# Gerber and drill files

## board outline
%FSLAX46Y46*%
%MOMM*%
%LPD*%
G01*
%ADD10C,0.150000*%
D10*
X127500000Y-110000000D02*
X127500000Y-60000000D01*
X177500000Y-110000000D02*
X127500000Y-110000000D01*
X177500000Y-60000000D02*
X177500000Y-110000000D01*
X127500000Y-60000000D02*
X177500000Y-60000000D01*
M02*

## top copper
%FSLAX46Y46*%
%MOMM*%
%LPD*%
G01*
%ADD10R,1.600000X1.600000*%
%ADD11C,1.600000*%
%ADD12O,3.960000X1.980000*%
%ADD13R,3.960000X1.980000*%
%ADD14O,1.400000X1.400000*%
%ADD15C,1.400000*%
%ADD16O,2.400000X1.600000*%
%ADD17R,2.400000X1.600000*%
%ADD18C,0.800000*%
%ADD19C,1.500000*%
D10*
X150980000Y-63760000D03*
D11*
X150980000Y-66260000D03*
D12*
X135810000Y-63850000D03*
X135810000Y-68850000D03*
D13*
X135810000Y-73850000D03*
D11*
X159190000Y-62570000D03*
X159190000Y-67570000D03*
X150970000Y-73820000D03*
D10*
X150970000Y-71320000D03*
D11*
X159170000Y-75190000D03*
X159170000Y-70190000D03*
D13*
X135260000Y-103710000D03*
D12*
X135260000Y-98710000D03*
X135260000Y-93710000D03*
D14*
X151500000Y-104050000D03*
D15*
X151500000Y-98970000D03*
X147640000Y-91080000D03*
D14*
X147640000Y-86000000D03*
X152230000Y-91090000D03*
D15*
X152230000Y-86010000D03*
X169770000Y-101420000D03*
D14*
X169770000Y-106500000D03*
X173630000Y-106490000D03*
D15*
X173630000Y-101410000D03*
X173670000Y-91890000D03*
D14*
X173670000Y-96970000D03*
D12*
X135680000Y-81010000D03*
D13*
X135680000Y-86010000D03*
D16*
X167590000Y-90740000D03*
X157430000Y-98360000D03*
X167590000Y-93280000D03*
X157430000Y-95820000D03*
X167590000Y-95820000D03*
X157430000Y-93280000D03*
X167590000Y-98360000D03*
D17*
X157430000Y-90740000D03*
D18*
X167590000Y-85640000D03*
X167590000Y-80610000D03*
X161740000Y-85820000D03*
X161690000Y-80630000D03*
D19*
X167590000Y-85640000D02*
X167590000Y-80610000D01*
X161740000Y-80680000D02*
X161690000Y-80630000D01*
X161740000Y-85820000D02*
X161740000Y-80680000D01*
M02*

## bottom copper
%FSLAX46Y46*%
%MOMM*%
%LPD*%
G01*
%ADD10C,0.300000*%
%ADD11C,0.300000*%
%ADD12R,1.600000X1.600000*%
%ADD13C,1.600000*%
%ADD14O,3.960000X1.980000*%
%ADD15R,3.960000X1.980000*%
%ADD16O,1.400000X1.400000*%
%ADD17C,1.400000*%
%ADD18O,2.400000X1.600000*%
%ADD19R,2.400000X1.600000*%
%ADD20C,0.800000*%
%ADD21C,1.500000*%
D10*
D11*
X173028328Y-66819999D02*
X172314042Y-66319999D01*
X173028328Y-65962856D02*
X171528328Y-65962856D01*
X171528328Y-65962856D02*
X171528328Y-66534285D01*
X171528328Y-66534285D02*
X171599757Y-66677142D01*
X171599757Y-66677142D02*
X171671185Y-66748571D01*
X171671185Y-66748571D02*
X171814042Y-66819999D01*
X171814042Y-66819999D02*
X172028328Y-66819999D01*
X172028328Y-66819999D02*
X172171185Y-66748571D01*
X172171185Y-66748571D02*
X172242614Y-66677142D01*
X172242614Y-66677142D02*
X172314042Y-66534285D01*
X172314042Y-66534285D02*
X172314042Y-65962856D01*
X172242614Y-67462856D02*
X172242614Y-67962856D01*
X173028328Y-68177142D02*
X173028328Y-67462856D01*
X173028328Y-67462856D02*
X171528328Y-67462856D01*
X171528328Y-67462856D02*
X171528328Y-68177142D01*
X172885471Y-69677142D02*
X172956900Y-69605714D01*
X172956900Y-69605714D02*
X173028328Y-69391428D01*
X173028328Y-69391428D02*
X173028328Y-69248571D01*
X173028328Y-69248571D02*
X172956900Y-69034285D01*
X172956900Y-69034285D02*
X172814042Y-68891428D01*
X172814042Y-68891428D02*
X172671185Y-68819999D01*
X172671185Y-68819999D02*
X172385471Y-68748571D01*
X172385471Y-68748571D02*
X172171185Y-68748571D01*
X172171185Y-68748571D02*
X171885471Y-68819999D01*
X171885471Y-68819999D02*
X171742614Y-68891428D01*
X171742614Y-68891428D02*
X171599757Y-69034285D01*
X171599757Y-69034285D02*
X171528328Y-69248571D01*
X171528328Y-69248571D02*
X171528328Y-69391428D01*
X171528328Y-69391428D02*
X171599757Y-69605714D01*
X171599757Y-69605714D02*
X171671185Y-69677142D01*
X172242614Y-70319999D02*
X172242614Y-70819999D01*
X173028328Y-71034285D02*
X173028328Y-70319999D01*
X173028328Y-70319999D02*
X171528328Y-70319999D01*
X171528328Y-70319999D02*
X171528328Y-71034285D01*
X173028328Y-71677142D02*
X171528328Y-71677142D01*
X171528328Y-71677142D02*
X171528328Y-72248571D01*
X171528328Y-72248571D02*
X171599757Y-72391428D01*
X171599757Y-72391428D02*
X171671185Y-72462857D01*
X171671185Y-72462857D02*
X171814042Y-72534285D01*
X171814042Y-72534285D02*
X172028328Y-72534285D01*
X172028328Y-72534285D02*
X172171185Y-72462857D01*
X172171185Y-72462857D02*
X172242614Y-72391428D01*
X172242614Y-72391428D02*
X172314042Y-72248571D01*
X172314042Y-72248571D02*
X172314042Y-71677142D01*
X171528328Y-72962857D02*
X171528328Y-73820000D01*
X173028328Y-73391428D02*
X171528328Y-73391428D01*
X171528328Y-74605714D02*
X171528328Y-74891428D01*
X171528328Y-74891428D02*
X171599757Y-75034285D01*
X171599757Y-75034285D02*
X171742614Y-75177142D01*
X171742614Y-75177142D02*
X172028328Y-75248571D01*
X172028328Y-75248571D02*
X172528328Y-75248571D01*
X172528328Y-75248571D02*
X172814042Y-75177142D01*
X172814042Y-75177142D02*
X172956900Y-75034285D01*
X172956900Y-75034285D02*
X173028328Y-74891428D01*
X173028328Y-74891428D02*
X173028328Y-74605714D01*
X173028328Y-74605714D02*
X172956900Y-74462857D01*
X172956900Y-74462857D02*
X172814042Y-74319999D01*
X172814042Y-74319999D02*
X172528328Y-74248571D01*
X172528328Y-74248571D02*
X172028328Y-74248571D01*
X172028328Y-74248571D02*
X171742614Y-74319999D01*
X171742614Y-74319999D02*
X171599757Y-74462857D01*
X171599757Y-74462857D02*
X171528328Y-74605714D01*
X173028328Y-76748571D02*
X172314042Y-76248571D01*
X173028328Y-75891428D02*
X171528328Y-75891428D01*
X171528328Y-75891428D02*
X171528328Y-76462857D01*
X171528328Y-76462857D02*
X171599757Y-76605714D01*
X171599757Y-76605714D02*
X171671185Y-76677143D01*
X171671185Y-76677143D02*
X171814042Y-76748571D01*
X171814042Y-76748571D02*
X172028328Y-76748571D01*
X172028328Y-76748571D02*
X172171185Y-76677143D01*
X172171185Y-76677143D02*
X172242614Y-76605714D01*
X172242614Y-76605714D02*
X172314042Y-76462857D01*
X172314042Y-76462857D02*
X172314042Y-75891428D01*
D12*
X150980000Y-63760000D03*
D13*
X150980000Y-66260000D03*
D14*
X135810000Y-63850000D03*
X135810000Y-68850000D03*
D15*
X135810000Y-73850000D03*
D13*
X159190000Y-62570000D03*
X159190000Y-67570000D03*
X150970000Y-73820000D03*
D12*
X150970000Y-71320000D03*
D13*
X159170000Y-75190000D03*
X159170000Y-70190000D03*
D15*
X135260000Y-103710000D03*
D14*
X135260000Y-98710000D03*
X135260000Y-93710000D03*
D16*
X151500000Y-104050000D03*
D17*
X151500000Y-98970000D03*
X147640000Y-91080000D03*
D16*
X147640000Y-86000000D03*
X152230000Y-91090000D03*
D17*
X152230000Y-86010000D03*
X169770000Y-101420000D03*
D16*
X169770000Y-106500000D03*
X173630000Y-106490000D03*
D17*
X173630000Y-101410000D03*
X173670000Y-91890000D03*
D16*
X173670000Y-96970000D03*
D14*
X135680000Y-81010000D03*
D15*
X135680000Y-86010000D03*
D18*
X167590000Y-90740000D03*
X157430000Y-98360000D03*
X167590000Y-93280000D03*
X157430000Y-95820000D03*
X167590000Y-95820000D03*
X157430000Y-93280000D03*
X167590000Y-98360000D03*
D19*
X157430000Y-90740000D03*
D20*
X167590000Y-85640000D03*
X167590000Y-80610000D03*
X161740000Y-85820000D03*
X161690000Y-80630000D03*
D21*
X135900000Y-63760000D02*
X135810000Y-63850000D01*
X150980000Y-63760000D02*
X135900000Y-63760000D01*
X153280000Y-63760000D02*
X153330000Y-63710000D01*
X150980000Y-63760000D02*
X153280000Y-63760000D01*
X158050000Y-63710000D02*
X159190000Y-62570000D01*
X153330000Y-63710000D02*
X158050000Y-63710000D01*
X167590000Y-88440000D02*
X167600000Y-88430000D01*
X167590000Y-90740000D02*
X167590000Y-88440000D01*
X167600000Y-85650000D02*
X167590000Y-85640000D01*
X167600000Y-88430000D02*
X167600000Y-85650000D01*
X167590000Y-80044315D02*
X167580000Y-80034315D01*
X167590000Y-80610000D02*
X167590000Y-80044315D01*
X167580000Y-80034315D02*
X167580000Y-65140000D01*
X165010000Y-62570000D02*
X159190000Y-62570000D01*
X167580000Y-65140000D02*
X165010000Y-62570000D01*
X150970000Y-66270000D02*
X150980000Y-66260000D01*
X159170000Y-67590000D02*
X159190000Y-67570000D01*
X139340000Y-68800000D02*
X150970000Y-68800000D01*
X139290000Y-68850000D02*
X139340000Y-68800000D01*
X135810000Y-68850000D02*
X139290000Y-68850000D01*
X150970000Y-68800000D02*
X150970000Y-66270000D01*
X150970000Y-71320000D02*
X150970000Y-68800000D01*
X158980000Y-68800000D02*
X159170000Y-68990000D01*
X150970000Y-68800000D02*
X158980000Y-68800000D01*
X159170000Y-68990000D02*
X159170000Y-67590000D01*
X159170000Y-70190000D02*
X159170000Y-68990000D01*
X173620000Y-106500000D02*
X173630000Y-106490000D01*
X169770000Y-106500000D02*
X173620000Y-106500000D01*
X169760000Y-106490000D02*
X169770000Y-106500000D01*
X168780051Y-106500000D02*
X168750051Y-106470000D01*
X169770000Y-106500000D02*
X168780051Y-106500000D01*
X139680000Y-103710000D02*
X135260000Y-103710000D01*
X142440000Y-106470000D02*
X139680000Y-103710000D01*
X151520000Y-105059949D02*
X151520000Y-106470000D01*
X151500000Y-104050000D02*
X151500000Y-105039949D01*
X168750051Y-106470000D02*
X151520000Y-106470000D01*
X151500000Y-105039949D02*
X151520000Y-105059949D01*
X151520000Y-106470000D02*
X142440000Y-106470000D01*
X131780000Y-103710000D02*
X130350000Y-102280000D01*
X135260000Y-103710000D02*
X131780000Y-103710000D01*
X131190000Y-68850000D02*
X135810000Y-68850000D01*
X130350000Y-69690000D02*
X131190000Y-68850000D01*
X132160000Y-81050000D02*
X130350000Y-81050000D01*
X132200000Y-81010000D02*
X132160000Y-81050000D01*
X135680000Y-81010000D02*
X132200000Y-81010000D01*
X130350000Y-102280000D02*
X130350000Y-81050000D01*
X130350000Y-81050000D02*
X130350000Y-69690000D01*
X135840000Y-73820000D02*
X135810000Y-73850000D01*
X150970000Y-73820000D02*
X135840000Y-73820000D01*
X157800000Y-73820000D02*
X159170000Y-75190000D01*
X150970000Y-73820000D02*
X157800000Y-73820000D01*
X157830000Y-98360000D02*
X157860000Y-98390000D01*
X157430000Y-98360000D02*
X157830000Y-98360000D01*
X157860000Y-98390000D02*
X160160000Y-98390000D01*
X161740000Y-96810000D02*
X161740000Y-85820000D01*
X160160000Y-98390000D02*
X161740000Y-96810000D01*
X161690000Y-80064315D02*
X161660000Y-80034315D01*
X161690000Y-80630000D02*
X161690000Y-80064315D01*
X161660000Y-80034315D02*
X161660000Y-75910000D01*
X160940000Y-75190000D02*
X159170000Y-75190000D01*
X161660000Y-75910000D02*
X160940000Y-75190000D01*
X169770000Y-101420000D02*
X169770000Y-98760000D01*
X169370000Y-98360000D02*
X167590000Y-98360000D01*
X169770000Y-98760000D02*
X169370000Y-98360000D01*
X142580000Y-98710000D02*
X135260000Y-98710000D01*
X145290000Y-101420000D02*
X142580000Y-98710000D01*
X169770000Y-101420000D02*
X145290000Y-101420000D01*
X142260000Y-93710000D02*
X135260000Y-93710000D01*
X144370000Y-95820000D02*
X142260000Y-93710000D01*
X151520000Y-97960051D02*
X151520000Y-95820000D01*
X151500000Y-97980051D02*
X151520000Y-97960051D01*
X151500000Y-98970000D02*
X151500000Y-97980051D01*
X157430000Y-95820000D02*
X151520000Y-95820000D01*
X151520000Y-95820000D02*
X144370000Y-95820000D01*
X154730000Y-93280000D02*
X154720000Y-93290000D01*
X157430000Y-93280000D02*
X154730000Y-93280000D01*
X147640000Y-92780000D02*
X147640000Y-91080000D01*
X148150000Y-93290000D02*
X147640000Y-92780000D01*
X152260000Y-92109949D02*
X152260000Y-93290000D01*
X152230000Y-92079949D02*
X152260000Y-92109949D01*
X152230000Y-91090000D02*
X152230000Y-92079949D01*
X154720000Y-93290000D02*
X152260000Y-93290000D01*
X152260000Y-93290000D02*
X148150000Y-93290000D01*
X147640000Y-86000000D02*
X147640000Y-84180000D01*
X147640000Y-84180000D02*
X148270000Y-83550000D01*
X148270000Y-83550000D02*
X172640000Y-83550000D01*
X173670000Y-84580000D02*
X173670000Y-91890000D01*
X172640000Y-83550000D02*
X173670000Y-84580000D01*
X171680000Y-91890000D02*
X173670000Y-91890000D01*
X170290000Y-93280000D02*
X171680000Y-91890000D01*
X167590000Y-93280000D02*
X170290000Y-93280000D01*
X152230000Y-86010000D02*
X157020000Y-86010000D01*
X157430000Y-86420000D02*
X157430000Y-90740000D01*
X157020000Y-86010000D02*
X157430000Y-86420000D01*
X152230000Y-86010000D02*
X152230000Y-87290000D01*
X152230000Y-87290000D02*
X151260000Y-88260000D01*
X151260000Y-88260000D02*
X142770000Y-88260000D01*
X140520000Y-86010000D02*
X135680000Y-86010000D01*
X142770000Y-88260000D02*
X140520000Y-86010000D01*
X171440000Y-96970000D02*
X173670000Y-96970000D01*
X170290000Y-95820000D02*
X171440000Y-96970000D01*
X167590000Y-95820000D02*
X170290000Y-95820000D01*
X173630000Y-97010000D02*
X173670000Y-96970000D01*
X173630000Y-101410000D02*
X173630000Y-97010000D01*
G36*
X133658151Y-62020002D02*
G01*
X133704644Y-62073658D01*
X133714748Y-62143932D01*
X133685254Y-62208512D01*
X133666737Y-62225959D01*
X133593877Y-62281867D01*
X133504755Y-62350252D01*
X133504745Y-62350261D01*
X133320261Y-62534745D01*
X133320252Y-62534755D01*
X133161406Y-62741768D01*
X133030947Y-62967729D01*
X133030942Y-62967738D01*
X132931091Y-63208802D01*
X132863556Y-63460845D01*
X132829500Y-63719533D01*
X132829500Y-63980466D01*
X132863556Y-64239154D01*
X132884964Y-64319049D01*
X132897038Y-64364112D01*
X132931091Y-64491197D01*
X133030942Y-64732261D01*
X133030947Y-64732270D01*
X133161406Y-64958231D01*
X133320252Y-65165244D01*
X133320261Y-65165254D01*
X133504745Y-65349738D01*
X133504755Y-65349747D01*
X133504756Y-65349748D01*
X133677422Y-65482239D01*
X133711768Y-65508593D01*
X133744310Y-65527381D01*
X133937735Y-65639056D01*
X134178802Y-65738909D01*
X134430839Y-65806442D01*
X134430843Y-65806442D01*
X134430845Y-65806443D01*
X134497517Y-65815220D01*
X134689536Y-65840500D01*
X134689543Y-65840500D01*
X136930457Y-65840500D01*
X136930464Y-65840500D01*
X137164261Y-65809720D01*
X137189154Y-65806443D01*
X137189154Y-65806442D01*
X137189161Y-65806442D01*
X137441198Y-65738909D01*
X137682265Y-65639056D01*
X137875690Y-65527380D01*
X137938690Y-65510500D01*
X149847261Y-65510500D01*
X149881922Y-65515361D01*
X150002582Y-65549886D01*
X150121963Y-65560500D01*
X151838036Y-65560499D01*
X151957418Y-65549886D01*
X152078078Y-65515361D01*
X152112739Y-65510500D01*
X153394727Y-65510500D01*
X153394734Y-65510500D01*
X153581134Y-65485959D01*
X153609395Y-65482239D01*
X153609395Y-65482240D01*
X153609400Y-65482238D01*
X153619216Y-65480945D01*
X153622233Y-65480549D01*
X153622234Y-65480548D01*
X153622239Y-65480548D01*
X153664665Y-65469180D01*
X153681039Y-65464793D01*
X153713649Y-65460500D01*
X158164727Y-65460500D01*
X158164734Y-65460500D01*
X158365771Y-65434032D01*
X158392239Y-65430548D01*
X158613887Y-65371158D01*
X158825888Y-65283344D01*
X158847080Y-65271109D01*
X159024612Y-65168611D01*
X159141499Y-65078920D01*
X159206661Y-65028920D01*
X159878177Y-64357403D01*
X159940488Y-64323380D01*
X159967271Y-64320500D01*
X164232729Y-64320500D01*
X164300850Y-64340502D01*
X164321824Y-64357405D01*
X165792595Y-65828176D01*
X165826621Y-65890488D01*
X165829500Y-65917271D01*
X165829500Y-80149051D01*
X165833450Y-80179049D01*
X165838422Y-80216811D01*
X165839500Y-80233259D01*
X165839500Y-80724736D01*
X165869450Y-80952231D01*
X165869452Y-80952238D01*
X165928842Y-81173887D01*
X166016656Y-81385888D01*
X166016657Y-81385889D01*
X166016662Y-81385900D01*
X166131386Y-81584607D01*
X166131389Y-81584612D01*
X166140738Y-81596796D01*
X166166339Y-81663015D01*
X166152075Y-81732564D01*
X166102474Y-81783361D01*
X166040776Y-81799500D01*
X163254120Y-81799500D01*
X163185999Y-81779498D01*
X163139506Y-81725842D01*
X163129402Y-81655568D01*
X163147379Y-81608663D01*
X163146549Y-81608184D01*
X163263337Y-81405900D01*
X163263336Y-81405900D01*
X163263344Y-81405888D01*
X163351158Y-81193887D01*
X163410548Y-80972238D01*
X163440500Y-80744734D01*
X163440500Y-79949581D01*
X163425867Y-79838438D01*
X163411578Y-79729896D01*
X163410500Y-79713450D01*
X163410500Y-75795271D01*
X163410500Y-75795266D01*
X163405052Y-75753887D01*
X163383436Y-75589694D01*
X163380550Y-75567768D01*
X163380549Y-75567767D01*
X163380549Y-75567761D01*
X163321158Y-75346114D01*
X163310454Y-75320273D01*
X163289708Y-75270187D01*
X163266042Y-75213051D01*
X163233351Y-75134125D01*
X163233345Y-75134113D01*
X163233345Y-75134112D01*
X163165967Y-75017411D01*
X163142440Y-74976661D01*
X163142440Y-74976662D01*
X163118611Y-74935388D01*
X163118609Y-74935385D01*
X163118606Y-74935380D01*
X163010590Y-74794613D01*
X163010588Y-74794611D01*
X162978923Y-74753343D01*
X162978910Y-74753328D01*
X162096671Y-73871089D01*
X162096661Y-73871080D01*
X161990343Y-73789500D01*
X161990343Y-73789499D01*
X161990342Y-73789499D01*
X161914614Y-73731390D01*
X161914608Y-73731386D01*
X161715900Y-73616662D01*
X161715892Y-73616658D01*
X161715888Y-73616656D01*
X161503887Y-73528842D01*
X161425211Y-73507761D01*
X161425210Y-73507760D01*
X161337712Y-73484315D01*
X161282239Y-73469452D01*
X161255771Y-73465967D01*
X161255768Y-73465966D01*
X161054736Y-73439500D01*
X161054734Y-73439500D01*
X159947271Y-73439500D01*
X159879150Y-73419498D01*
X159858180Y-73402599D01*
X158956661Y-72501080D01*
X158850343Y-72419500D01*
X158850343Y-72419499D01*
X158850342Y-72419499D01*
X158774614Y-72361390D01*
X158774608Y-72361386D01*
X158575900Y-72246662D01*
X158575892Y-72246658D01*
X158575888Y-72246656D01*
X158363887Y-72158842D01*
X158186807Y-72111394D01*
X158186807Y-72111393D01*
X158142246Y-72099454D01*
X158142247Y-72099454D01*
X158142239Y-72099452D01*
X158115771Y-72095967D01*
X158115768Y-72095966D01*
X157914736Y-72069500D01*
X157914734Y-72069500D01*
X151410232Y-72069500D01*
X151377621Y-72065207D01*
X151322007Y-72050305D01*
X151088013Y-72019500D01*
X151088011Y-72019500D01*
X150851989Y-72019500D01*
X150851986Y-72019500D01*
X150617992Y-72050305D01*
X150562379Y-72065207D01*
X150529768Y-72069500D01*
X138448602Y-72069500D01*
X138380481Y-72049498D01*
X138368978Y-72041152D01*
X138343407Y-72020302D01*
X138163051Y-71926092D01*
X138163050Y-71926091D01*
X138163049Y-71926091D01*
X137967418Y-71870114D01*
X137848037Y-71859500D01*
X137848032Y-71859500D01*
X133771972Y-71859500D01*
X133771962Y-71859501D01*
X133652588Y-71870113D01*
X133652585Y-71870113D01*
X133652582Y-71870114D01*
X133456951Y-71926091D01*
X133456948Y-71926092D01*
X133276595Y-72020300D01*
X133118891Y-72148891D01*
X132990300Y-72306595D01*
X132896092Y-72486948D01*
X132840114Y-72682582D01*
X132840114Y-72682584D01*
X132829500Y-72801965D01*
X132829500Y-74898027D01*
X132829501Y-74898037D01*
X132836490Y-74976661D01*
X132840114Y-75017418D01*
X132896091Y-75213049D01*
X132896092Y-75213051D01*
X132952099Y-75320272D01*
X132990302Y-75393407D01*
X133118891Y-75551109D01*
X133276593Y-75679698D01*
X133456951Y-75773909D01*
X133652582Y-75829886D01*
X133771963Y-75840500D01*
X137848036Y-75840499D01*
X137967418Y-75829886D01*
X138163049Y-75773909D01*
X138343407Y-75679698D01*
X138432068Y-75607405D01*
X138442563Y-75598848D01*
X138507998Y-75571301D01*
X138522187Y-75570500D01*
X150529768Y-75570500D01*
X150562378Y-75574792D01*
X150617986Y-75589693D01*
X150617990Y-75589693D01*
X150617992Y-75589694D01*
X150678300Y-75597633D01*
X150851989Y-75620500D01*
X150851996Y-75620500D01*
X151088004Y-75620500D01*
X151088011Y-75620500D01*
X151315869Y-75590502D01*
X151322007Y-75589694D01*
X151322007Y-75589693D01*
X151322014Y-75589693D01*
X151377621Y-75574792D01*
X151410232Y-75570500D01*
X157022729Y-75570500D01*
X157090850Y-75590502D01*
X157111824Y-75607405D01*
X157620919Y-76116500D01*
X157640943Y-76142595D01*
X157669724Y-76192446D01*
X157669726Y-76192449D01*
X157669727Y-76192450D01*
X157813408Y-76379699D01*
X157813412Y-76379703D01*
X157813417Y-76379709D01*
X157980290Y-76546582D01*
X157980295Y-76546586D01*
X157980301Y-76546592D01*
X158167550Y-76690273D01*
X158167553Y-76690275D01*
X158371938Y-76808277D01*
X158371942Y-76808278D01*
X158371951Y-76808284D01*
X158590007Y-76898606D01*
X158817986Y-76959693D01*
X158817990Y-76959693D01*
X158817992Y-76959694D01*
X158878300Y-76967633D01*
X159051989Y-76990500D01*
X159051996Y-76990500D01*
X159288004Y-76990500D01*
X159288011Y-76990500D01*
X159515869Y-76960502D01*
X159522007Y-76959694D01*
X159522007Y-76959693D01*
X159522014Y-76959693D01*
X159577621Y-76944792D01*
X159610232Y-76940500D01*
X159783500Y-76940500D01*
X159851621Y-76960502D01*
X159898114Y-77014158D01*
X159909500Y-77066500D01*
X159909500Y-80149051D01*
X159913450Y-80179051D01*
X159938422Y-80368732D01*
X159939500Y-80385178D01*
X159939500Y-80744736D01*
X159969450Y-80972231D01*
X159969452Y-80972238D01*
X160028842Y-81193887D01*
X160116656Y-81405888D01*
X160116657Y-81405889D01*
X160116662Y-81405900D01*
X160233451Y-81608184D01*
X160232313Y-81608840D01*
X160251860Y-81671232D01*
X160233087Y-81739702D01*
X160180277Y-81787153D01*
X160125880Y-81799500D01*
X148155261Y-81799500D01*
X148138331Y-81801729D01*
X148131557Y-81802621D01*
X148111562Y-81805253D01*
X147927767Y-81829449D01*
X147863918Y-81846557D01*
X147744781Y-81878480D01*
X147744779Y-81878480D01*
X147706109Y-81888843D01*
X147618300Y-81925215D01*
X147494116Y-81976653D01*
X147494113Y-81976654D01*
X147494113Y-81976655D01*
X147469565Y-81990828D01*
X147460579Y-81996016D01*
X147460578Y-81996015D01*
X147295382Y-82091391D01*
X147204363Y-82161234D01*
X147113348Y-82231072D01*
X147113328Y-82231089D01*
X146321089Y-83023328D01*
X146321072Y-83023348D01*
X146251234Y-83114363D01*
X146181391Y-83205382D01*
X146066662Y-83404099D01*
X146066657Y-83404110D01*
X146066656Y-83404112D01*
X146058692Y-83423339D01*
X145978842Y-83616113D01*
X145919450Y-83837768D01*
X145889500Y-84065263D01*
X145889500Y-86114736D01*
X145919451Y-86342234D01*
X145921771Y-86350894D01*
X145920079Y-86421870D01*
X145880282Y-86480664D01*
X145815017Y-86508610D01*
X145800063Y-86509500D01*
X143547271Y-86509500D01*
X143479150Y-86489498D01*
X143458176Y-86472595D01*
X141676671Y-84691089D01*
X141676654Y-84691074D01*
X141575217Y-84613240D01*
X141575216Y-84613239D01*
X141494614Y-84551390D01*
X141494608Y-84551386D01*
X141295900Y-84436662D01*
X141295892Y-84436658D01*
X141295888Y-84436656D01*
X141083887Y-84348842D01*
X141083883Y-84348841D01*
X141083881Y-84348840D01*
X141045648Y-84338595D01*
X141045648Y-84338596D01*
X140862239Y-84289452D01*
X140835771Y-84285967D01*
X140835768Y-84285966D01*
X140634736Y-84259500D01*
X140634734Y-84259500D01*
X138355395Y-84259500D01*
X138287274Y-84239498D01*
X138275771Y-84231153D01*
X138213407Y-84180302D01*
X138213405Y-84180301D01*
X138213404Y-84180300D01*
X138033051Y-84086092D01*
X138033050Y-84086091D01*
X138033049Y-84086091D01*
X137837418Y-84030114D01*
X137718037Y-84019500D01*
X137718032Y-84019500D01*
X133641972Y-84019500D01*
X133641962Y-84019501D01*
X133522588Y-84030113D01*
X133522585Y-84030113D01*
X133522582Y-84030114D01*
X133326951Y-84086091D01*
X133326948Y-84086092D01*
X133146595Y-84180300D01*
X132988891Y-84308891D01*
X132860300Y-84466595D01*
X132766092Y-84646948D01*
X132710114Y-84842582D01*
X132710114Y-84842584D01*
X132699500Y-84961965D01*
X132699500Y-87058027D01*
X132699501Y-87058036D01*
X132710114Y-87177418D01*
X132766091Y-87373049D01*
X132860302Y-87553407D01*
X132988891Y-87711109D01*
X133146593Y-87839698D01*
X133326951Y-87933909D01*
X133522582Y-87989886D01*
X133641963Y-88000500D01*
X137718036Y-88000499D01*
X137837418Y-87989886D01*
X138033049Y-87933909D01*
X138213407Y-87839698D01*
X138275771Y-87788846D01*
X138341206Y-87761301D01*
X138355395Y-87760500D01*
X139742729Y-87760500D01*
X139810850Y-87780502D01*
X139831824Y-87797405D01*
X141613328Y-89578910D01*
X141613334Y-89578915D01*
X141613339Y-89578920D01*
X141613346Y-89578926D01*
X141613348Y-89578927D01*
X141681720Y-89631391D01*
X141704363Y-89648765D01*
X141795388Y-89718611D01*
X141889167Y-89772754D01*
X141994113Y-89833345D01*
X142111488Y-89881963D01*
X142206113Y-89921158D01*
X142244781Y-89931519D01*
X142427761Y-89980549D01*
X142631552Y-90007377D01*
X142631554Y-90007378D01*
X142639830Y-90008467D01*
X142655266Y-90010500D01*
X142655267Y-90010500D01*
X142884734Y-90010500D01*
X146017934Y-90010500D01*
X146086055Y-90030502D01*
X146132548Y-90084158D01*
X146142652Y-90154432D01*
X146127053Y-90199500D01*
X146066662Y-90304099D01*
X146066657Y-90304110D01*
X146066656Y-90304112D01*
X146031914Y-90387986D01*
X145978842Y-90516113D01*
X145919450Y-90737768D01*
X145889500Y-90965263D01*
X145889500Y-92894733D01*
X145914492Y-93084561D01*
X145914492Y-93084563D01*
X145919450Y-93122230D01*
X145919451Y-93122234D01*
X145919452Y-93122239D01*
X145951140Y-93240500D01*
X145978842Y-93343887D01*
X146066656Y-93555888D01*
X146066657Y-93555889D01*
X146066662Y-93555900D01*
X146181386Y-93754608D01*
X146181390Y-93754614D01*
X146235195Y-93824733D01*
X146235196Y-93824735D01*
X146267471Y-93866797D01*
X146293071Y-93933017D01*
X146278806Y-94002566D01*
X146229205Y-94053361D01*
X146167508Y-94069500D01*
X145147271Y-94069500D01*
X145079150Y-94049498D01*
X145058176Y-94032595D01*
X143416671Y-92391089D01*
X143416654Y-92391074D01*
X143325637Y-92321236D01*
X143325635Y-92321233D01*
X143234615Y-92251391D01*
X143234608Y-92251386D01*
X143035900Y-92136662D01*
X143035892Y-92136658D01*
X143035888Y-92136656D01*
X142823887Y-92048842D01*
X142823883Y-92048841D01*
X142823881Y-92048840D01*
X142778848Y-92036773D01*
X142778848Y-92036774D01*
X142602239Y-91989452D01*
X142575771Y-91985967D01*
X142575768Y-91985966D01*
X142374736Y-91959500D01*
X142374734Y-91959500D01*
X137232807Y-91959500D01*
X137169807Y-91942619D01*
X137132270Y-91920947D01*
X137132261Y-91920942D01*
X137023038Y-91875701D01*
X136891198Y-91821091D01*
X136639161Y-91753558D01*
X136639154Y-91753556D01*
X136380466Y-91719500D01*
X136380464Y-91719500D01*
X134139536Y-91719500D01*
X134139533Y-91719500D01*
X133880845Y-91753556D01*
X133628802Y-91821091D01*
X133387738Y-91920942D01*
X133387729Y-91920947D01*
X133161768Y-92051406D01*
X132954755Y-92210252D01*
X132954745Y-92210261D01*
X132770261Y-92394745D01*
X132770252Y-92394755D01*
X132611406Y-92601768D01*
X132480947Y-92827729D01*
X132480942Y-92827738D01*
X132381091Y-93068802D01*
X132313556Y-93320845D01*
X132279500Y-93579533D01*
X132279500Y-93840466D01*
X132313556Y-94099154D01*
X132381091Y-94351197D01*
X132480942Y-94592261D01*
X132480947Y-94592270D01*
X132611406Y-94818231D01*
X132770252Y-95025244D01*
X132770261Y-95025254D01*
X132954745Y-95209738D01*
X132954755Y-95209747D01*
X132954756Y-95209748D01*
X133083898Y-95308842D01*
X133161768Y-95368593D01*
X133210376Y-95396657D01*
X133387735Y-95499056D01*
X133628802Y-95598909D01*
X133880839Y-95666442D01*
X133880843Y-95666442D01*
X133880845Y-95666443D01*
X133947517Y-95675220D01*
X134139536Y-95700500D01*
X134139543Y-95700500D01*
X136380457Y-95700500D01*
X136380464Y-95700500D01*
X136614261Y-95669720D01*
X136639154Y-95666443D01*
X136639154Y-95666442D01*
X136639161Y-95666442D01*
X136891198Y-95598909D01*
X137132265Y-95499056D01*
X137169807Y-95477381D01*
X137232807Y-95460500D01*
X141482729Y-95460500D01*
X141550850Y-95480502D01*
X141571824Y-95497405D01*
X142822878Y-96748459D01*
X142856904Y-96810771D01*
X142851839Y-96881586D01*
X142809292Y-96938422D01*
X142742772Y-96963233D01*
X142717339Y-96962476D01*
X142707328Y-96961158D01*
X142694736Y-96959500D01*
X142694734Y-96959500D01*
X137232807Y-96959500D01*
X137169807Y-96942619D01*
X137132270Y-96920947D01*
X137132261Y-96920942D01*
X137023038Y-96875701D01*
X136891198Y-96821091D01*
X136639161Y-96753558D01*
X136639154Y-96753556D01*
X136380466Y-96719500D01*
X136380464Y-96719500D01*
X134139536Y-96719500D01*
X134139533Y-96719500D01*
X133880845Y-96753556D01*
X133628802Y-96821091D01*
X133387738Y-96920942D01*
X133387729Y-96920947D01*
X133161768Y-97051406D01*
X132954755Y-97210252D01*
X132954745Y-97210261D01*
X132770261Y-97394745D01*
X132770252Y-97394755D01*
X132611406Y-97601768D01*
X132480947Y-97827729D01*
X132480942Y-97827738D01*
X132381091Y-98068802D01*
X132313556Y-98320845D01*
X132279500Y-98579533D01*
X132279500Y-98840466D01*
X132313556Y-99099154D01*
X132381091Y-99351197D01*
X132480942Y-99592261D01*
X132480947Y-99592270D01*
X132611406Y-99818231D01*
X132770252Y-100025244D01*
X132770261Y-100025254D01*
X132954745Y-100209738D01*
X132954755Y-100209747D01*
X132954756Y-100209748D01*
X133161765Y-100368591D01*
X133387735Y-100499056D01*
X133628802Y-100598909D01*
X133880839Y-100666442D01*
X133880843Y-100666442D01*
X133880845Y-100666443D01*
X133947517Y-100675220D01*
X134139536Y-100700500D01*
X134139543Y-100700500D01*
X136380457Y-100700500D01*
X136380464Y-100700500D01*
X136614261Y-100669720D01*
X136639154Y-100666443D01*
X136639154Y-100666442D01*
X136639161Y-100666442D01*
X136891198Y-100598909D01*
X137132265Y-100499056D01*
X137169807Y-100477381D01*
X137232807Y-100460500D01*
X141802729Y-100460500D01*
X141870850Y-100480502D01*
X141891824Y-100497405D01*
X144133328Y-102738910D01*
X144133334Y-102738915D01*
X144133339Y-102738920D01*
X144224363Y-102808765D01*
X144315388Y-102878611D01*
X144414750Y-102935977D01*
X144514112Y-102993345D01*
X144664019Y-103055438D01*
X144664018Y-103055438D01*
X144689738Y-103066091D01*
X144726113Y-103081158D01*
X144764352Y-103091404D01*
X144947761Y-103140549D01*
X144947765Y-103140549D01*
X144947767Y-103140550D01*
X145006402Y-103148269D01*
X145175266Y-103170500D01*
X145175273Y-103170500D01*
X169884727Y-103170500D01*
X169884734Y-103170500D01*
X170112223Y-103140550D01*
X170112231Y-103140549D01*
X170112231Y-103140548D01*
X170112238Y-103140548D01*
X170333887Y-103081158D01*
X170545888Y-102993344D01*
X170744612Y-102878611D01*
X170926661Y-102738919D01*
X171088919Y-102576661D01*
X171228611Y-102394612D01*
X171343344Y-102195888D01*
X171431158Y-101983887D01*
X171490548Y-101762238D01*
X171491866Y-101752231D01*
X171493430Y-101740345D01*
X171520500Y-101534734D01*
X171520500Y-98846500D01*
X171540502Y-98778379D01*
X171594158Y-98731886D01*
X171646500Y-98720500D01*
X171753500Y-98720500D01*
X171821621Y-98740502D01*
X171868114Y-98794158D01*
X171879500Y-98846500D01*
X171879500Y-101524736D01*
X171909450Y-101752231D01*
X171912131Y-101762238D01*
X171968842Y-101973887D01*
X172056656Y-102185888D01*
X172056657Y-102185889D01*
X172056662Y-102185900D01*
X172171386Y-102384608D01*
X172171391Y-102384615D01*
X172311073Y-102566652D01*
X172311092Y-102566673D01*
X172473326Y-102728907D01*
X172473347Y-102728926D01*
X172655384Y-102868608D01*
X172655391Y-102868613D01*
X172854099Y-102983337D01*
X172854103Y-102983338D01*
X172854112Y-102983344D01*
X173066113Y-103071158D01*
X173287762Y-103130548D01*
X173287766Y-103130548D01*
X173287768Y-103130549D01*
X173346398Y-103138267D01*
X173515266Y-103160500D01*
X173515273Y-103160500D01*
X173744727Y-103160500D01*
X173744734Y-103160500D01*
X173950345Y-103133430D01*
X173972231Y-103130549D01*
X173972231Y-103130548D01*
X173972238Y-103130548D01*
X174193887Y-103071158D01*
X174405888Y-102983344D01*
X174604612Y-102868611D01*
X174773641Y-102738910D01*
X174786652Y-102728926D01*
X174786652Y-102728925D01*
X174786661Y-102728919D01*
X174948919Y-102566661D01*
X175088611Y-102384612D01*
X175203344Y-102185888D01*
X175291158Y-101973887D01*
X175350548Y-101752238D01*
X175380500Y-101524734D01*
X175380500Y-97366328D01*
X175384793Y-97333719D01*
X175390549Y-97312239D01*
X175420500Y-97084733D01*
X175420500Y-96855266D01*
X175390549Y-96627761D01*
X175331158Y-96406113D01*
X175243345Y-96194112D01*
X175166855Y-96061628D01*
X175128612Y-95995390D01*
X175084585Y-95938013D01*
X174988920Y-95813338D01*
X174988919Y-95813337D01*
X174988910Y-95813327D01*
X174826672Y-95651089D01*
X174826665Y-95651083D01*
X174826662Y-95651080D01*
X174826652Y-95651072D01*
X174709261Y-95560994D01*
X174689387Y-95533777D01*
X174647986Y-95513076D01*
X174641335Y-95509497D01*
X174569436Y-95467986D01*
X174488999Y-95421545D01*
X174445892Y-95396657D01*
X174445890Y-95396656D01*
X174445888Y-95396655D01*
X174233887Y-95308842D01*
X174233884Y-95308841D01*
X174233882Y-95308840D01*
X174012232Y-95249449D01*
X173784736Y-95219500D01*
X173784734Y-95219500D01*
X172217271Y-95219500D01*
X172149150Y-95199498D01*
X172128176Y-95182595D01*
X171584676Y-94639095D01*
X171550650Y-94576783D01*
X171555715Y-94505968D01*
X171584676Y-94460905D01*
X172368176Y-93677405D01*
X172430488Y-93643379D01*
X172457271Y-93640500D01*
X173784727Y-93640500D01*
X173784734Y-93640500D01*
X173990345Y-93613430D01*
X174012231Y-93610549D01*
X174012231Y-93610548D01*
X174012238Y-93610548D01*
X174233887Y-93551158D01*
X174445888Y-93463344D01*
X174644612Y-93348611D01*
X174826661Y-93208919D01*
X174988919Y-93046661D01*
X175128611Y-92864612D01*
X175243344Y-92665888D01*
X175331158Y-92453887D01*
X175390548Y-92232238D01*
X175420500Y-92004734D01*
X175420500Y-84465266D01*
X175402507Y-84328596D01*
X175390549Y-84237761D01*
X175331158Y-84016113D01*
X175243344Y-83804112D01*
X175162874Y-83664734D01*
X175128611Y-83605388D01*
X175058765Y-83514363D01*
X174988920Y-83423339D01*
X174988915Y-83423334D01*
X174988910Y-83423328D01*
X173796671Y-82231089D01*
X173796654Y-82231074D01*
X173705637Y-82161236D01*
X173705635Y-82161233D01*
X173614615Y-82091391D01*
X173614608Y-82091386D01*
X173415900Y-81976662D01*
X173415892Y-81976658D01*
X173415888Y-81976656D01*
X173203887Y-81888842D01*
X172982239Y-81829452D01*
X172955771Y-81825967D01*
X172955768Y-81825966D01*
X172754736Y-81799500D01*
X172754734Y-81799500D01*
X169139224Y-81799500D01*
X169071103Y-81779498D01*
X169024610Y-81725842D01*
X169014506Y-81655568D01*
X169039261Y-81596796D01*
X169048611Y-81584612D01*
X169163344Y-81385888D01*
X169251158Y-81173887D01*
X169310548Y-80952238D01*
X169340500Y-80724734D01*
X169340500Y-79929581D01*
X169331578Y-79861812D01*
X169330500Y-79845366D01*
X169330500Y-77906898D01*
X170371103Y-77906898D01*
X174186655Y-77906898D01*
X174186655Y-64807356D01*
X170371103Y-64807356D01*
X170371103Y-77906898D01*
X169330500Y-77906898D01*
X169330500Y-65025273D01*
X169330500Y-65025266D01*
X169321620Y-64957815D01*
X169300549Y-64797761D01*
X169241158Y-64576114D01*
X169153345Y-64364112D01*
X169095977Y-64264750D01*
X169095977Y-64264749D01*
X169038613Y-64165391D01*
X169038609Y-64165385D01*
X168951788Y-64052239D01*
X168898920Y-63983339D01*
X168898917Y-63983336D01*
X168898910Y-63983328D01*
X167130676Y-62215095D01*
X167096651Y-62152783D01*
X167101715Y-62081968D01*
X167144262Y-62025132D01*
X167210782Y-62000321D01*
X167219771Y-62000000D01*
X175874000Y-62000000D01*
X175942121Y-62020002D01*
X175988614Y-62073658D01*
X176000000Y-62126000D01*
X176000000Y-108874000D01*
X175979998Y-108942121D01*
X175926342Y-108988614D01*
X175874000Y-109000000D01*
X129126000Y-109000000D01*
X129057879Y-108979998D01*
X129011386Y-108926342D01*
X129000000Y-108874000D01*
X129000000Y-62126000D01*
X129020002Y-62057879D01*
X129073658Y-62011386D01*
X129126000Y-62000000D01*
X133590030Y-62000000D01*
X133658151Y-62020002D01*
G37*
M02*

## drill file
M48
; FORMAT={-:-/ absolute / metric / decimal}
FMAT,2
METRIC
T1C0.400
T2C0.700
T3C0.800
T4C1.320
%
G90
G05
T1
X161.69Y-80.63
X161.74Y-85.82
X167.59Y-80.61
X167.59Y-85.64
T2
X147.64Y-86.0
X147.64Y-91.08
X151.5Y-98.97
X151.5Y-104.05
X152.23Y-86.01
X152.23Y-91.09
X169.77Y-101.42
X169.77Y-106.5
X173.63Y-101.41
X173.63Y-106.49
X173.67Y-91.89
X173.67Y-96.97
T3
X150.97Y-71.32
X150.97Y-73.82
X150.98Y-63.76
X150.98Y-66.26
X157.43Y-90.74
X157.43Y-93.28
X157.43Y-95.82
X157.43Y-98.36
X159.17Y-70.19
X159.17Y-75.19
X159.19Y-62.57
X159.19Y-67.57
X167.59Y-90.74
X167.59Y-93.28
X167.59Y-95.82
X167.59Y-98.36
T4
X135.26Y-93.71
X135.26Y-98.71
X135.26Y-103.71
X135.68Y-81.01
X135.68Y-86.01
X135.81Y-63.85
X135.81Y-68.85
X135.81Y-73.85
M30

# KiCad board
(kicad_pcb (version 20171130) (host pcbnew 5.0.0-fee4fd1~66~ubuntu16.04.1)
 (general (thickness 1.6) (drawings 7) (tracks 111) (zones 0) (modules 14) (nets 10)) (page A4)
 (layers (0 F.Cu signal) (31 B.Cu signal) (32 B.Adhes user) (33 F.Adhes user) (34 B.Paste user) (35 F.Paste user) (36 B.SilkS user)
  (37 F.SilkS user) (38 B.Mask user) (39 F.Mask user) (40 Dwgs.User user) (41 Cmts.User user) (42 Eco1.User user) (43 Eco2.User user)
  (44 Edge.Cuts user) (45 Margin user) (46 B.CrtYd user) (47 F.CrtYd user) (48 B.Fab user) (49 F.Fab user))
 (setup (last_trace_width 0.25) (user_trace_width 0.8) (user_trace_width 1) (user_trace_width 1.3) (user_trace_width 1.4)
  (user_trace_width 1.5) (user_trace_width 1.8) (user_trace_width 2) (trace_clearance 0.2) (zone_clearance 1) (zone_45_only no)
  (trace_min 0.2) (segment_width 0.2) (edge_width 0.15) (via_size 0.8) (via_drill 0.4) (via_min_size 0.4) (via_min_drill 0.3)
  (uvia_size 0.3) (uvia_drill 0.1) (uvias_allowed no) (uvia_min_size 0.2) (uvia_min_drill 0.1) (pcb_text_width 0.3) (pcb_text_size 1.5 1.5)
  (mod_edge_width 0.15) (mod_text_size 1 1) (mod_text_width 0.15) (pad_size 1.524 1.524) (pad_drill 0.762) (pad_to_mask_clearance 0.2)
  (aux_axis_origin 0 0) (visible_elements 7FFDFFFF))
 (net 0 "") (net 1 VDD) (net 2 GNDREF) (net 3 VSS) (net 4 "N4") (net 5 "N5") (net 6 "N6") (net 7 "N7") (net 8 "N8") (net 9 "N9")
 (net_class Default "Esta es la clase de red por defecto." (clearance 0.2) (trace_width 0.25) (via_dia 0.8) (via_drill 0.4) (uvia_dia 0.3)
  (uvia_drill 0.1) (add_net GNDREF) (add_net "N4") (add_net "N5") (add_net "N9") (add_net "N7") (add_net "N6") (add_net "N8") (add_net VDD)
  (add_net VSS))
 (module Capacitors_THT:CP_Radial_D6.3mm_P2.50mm (layer F.Cu) (at 150.98 63.76 270)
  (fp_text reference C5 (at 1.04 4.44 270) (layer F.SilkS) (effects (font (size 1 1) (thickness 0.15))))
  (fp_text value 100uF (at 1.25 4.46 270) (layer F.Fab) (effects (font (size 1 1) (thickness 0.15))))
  (pad 1 thru_hole rect (at 0 0 270) (size 1.6 1.6) (drill 0.8) (layers *.Cu *.Mask) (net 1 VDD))
  (pad 2 thru_hole circle (at 2.5 0 270) (size 1.6 1.6) (drill 0.8) (layers *.Cu *.Mask) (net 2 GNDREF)))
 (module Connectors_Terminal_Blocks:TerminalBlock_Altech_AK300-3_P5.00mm (layer F.Cu) (at 135.81 73.85 90)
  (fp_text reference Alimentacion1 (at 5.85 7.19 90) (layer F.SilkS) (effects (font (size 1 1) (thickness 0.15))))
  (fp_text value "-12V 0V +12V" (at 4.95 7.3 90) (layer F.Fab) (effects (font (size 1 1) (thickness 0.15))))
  (pad 3 thru_hole oval (at 10 0 90) (size 1.98 3.96) (drill 1.32) (layers *.Cu *.Mask) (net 1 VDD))
  (pad 2 thru_hole oval (at 5 0 90) (size 1.98 3.96) (drill 1.32) (layers *.Cu *.Mask) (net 2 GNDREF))
  (pad 1 thru_hole rect (at 0 0 90) (size 1.98 3.96) (drill 1.32) (layers *.Cu *.Mask) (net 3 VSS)))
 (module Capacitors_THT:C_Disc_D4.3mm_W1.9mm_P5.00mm (layer F.Cu) (at 159.19 67.57 90)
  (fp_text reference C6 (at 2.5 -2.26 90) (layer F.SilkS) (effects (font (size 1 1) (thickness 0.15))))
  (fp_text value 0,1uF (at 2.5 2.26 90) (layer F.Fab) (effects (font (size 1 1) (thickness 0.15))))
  (pad 2 thru_hole circle (at 5 0 90) (size 1.6 1.6) (drill 0.8) (layers *.Cu *.Mask) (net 1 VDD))
  (pad 1 thru_hole circle (at 0 0 90) (size 1.6 1.6) (drill 0.8) (layers *.Cu *.Mask) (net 2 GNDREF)))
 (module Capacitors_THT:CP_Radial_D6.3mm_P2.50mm (layer F.Cu) (at 150.97 71.32 270)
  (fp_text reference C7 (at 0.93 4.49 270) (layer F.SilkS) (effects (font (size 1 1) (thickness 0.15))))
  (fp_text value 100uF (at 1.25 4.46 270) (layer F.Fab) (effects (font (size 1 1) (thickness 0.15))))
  (pad 2 thru_hole circle (at 2.5 0 270) (size 1.6 1.6) (drill 0.8) (layers *.Cu *.Mask) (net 3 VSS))
  (pad 1 thru_hole rect (at 0 0 270) (size 1.6 1.6) (drill 0.8) (layers *.Cu *.Mask) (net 2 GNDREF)))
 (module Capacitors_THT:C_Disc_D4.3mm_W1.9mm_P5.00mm (layer F.Cu) (at 159.17 75.19 90)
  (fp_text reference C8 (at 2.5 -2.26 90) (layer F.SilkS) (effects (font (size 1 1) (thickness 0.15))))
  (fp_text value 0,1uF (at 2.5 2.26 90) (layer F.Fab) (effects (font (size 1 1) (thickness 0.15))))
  (pad 1 thru_hole circle (at 0 0 90) (size 1.6 1.6) (drill 0.8) (layers *.Cu *.Mask) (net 3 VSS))
  (pad 2 thru_hole circle (at 5 0 90) (size 1.6 1.6) (drill 0.8) (layers *.Cu *.Mask) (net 2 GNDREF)))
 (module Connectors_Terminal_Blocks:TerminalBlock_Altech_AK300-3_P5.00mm (layer F.Cu) (at 135.26 103.71 90)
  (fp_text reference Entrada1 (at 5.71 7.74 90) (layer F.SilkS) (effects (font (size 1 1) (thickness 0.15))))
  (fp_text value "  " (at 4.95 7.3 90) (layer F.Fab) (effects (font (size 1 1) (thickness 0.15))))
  (pad 1 thru_hole rect (at 0 0 90) (size 1.98 3.96) (drill 1.32) (layers *.Cu *.Mask) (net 2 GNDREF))
  (pad 2 thru_hole oval (at 5 0 90) (size 1.98 3.96) (drill 1.32) (layers *.Cu *.Mask) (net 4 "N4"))
  (pad 3 thru_hole oval (at 10 0 90) (size 1.98 3.96) (drill 1.32) (layers *.Cu *.Mask) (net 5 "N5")))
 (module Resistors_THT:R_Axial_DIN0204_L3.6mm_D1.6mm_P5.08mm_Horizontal (layer F.Cu) (at 151.5 98.97 270)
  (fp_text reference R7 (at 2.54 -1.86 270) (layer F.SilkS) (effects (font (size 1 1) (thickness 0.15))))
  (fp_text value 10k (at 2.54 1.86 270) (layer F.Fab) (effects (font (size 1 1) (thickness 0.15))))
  (pad 2 thru_hole oval (at 5.08 0 270) (size 1.4 1.4) (drill 0.7) (layers *.Cu *.Mask) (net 2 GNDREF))
  (pad 1 thru_hole circle (at 0 0 270) (size 1.4 1.4) (drill 0.7) (layers *.Cu *.Mask) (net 5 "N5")))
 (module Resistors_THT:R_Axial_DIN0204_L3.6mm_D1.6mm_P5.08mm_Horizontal (layer F.Cu) (at 147.64 91.08 90)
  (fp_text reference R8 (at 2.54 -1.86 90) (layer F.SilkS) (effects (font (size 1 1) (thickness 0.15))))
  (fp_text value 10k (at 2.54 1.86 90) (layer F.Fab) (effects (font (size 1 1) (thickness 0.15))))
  (pad 1 thru_hole circle (at 0 0 90) (size 1.4 1.4) (drill 0.7) (layers *.Cu *.Mask) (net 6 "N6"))
  (pad 2 thru_hole oval (at 5.08 0 90) (size 1.4 1.4) (drill 0.7) (layers *.Cu *.Mask) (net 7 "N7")))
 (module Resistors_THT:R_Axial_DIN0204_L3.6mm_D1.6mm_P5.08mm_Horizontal (layer F.Cu) (at 152.23 86.01 270)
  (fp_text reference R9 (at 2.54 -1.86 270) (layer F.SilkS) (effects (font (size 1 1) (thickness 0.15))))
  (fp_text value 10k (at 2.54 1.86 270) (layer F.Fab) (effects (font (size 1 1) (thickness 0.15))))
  (pad 2 thru_hole oval (at 5.08 0 270) (size 1.4 1.4) (drill 0.7) (layers *.Cu *.Mask) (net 6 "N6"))
  (pad 1 thru_hole circle (at 0 0 270) (size 1.4 1.4) (drill 0.7) (layers *.Cu *.Mask) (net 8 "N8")))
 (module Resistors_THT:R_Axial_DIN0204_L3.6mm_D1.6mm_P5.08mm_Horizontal (layer F.Cu) (at 169.77 101.42 270)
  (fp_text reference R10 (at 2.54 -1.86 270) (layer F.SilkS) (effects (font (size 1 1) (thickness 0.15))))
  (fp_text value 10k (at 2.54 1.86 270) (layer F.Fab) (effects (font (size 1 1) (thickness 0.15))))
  (pad 1 thru_hole circle (at 0 0 270) (size 1.4 1.4) (drill 0.7) (layers *.Cu *.Mask) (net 4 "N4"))
  (pad 2 thru_hole oval (at 5.08 0 270) (size 1.4 1.4) (drill 0.7) (layers *.Cu *.Mask) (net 2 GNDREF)))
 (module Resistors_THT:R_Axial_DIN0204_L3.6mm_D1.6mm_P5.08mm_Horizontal (layer F.Cu) (at 173.63 101.41 270)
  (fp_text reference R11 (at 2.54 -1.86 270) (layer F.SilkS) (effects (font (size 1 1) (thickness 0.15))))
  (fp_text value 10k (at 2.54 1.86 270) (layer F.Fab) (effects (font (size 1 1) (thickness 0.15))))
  (pad 2 thru_hole oval (at 5.08 0 270) (size 1.4 1.4) (drill 0.7) (layers *.Cu *.Mask) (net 2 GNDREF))
  (pad 1 thru_hole circle (at 0 0 270) (size 1.4 1.4) (drill 0.7) (layers *.Cu *.Mask) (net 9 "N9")))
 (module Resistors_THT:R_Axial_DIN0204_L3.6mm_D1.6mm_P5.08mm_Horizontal (layer F.Cu) (at 173.67 91.89 270)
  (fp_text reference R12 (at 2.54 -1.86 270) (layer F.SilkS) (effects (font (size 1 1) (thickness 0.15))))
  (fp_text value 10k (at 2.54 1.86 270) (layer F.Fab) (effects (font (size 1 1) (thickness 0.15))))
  (pad 1 thru_hole circle (at 0 0 270) (size 1.4 1.4) (drill 0.7) (layers *.Cu *.Mask) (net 7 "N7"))
  (pad 2 thru_hole oval (at 5.08 0 270) (size 1.4 1.4) (drill 0.7) (layers *.Cu *.Mask) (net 9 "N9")))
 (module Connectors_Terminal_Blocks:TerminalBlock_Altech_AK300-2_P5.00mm (layer F.Cu) (at 135.68 86.01 90)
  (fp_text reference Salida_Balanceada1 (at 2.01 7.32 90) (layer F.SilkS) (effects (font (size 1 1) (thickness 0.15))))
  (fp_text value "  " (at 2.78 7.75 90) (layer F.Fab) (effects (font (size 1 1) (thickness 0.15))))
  (pad 2 thru_hole oval (at 5 0 90) (size 1.98 3.96) (drill 1.32) (layers *.Cu *.Mask) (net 2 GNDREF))
  (pad 1 thru_hole rect (at 0 0 90) (size 1.98 3.96) (drill 1.32) (layers *.Cu *.Mask) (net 8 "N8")))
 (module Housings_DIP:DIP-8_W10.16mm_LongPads (layer F.Cu) (at 157.43 90.74)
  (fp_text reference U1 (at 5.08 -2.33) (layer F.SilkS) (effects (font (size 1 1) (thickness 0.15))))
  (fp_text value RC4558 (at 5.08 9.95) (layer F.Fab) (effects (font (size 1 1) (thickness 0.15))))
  (pad 8 thru_hole oval (at 10.16 0) (size 2.4 1.6) (drill 0.8) (layers *.Cu *.Mask) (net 1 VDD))
  (pad 4 thru_hole oval (at 0 7.62) (size 2.4 1.6) (drill 0.8) (layers *.Cu *.Mask) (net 3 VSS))
  (pad 7 thru_hole oval (at 10.16 2.54) (size 2.4 1.6) (drill 0.8) (layers *.Cu *.Mask) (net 7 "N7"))
  (pad 3 thru_hole oval (at 0 5.08) (size 2.4 1.6) (drill 0.8) (layers *.Cu *.Mask) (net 5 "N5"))
  (pad 6 thru_hole oval (at 10.16 5.08) (size 2.4 1.6) (drill 0.8) (layers *.Cu *.Mask) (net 9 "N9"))
  (pad 2 thru_hole oval (at 0 2.54) (size 2.4 1.6) (drill 0.8) (layers *.Cu *.Mask) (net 6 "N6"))
  (pad 5 thru_hole oval (at 10.16 7.62) (size 2.4 1.6) (drill 0.8) (layers *.Cu *.Mask) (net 4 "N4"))
  (pad 1 thru_hole rect (at 0 0) (size 2.4 1.6) (drill 0.8) (layers *.Cu *.Mask) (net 8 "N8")))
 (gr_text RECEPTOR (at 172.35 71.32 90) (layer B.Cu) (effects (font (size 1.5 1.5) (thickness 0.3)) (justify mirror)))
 (gr_line (start 127.5 110) (end 127.5 60) (layer Edge.Cuts) (width 0.15))
 (gr_line (start 177.5 110) (end 127.5 110) (layer Edge.Cuts) (width 0.15))
 (gr_line (start 177.5 60) (end 177.5 110) (layer Edge.Cuts) (width 0.15))
 (gr_line (start 127.5 60) (end 177.5 60) (layer Edge.Cuts) (width 0.15))
 (segment (start 135.9 63.76) (end 135.81 63.85) (width 1.5) (layer B.Cu) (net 1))
 (segment (start 150.98 63.76) (end 135.9 63.76) (width 1.5) (layer B.Cu) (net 1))
 (segment (start 153.28 63.76) (end 153.33 63.71) (width 1.5) (layer B.Cu) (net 1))
 (segment (start 150.98 63.76) (end 153.28 63.76) (width 1.5) (layer B.Cu) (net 1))
 (segment (start 158.05 63.71) (end 159.19 62.57) (width 1.5) (layer B.Cu) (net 1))
 (segment (start 153.33 63.71) (end 158.05 63.71) (width 1.5) (layer B.Cu) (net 1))
 (segment (start 167.59 88.44) (end 167.6 88.43) (width 1.5) (layer B.Cu) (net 1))
 (segment (start 167.59 90.74) (end 167.59 88.44) (width 1.5) (layer B.Cu) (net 1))
 (via (at 167.59 85.64) (size 0.8) (drill 0.4) (layers F.Cu B.Cu) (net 1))
 (segment (start 167.6 85.65) (end 167.59 85.64) (width 1.5) (layer B.Cu) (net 1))
 (segment (start 167.6 88.43) (end 167.6 85.65) (width 1.5) (layer B.Cu) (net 1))
 (segment (start 167.59 85.64) (end 167.59 80.61) (width 1.5) (layer F.Cu) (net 1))
 (via (at 167.59 80.61) (size 0.8) (drill 0.4) (layers F.Cu B.Cu) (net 1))
 (segment (start 167.59 80.044315) (end 167.58 80.034315) (width 1.5) (layer B.Cu) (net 1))
 (segment (start 167.59 80.61) (end 167.59 80.044315) (width 1.5) (layer B.Cu) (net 1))
 (segment (start 167.58 80.034315) (end 167.58 65.14) (width 1.5) (layer B.Cu) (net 1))
 (segment (start 165.01 62.57) (end 159.19 62.57) (width 1.5) (layer B.Cu) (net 1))
 (segment (start 167.58 65.14) (end 165.01 62.57) (width 1.5) (layer B.Cu) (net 1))
 (segment (start 150.97 66.27) (end 150.98 66.26) (width 1.5) (layer B.Cu) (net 2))
 (segment (start 159.17 67.59) (end 159.19 67.57) (width 1.5) (layer B.Cu) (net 2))
 (segment (start 139.34 68.8) (end 150.97 68.8) (width 1.5) (layer B.Cu) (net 2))
 (segment (start 139.29 68.85) (end 139.34 68.8) (width 1.5) (layer B.Cu) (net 2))
 (segment (start 135.81 68.85) (end 139.29 68.85) (width 1.5) (layer B.Cu) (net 2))
 (segment (start 150.97 68.8) (end 150.97 66.27) (width 1.5) (layer B.Cu) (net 2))
 (segment (start 150.97 71.32) (end 150.97 68.8) (width 1.5) (layer B.Cu) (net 2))
 (segment (start 158.98 68.8) (end 159.17 68.99) (width 1.5) (layer B.Cu) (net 2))
 (segment (start 150.97 68.8) (end 158.98 68.8) (width 1.5) (layer B.Cu) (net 2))
 (segment (start 159.17 68.99) (end 159.17 67.59) (width 1.5) (layer B.Cu) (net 2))
 (segment (start 159.17 70.19) (end 159.17 68.99) (width 1.5) (layer B.Cu) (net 2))
 (segment (start 173.62 106.5) (end 173.63 106.49) (width 1.5) (layer B.Cu) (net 2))
 (segment (start 169.77 106.5) (end 173.62 106.5) (width 1.5) (layer B.Cu) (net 2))
 (segment (start 169.76 106.49) (end 169.77 106.5) (width 1.5) (layer B.Cu) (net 2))
 (segment (start 168.780051 106.5) (end 168.750051 106.47) (width 1.5) (layer B.Cu) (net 2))
 (segment (start 169.77 106.5) (end 168.780051 106.5) (width 1.5) (layer B.Cu) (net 2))
 (segment (start 139.68 103.71) (end 135.26 103.71) (width 1.5) (layer B.Cu) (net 2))
 (segment (start 142.44 106.47) (end 139.68 103.71) (width 1.5) (layer B.Cu) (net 2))
 (segment (start 151.52 105.059949) (end 151.52 106.47) (width 1.5) (layer B.Cu) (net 2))
 (segment (start 151.5 104.05) (end 151.5 105.039949) (width 1.5) (layer B.Cu) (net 2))
 (segment (start 168.750051 106.47) (end 151.52 106.47) (width 1.5) (layer B.Cu) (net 2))
 (segment (start 151.5 105.039949) (end 151.52 105.059949) (width 1.5) (layer B.Cu) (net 2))
 (segment (start 151.52 106.47) (end 142.44 106.47) (width 1.5) (layer B.Cu) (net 2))
 (segment (start 131.78 103.71) (end 130.35 102.28) (width 1.5) (layer B.Cu) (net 2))
 (segment (start 135.26 103.71) (end 131.78 103.71) (width 1.5) (layer B.Cu) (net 2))
 (segment (start 131.19 68.85) (end 135.81 68.85) (width 1.5) (layer B.Cu) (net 2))
 (segment (start 130.35 69.69) (end 131.19 68.85) (width 1.5) (layer B.Cu) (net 2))
 (segment (start 132.16 81.05) (end 130.35 81.05) (width 1.5) (layer B.Cu) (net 2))
 (segment (start 132.2 81.01) (end 132.16 81.05) (width 1.5) (layer B.Cu) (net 2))
 (segment (start 135.68 81.01) (end 132.2 81.01) (width 1.5) (layer B.Cu) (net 2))
 (segment (start 130.35 102.28) (end 130.35 81.05) (width 1.5) (layer B.Cu) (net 2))
 (segment (start 130.35 81.05) (end 130.35 69.69) (width 1.5) (layer B.Cu) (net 2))
 (segment (start 135.84 73.82) (end 135.81 73.85) (width 1.5) (layer B.Cu) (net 3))
 (segment (start 150.97 73.82) (end 135.84 73.82) (width 1.5) (layer B.Cu) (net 3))
 (segment (start 157.8 73.82) (end 159.17 75.19) (width 1.5) (layer B.Cu) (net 3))
 (segment (start 150.97 73.82) (end 157.8 73.82) (width 1.5) (layer B.Cu) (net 3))
 (segment (start 157.83 98.36) (end 157.86 98.39) (width 1.5) (layer B.Cu) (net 3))
 (segment (start 157.43 98.36) (end 157.83 98.36) (width 1.5) (layer B.Cu) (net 3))
 (segment (start 157.86 98.39) (end 160.16 98.39) (width 1.5) (layer B.Cu) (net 3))
 (segment (start 161.74 96.81) (end 161.74 85.82) (width 1.5) (layer B.Cu) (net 3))
 (via (at 161.74 85.82) (size 0.8) (drill 0.4) (layers F.Cu B.Cu) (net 3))
 (segment (start 160.16 98.39) (end 161.74 96.81) (width 1.5) (layer B.Cu) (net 3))
 (via (at 161.69 80.63) (size 0.8) (drill 0.4) (layers F.Cu B.Cu) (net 3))
 (segment (start 161.74 80.68) (end 161.69 80.63) (width 1.5) (layer F.Cu) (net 3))
 (segment (start 161.74 85.82) (end 161.74 80.68) (width 1.5) (layer F.Cu) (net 3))
 (segment (start 161.69 80.064315) (end 161.66 80.034315) (width 1.5) (layer B.Cu) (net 3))
 (segment (start 161.69 80.63) (end 161.69 80.064315) (width 1.5) (layer B.Cu) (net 3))
 (segment (start 161.66 80.034315) (end 161.66 75.91) (width 1.5) (layer B.Cu) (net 3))
 (segment (start 160.94 75.19) (end 159.17 75.19) (width 1.5) (layer B.Cu) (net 3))
 (segment (start 161.66 75.91) (end 160.94 75.19) (width 1.5) (layer B.Cu) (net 3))
 (segment (start 169.77 101.42) (end 169.77 98.76) (width 1.5) (layer B.Cu) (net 4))
 (segment (start 169.37 98.36) (end 167.59 98.36) (width 1.5) (layer B.Cu) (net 4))
 (segment (start 169.77 98.76) (end 169.37 98.36) (width 1.5) (layer B.Cu) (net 4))
 (segment (start 142.58 98.71) (end 135.26 98.71) (width 1.5) (layer B.Cu) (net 4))
 (segment (start 145.29 101.42) (end 142.58 98.71) (width 1.5) (layer B.Cu) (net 4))
 (segment (start 169.77 101.42) (end 145.29 101.42) (width 1.5) (layer B.Cu) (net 4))
 (segment (start 142.26 93.71) (end 135.26 93.71) (width 1.5) (layer B.Cu) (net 5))
 (segment (start 144.37 95.82) (end 142.26 93.71) (width 1.5) (layer B.Cu) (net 5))
 (segment (start 151.52 97.960051) (end 151.52 95.82) (width 1.5) (layer B.Cu) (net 5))
 (segment (start 151.5 97.980051) (end 151.52 97.960051) (width 1.5) (layer B.Cu) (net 5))
 (segment (start 151.5 98.97) (end 151.5 97.980051) (width 1.5) (layer B.Cu) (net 5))
 (segment (start 157.43 95.82) (end 151.52 95.82) (width 1.5) (layer B.Cu) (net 5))
 (segment (start 151.52 95.82) (end 144.37 95.82) (width 1.5) (layer B.Cu) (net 5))
 (segment (start 154.73 93.28) (end 154.72 93.29) (width 1.5) (layer B.Cu) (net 6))
 (segment (start 157.43 93.28) (end 154.73 93.28) (width 1.5) (layer B.Cu) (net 6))
 (segment (start 147.64 92.78) (end 147.64 91.08) (width 1.5) (layer B.Cu) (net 6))
 (segment (start 148.15 93.29) (end 147.64 92.78) (width 1.5) (layer B.Cu) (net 6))
 (segment (start 152.26 92.109949) (end 152.26 93.29) (width 1.5) (layer B.Cu) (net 6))
 (segment (start 152.23 92.079949) (end 152.26 92.109949) (width 1.5) (layer B.Cu) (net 6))
 (segment (start 152.23 91.09) (end 152.23 92.079949) (width 1.5) (layer B.Cu) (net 6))
 (segment (start 154.72 93.29) (end 152.26 93.29) (width 1.5) (layer B.Cu) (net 6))
 (segment (start 152.26 93.29) (end 148.15 93.29) (width 1.5) (layer B.Cu) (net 6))
 (segment (start 147.64 86) (end 147.64 84.18) (width 1.5) (layer B.Cu) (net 7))
 (segment (start 147.64 84.18) (end 148.27 83.55) (width 1.5) (layer B.Cu) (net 7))
 (segment (start 148.27 83.55) (end 172.64 83.55) (width 1.5) (layer B.Cu) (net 7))
 (segment (start 173.67 84.58) (end 173.67 91.89) (width 1.5) (layer B.Cu) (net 7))
 (segment (start 172.64 83.55) (end 173.67 84.58) (width 1.5) (layer B.Cu) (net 7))
 (segment (start 171.68 91.89) (end 173.67 91.89) (width 1.5) (layer B.Cu) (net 7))
 (segment (start 170.29 93.28) (end 171.68 91.89) (width 1.5) (layer B.Cu) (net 7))
 (segment (start 167.59 93.28) (end 170.29 93.28) (width 1.5) (layer B.Cu) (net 7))
 (segment (start 152.23 86.01) (end 157.02 86.01) (width 1.5) (layer B.Cu) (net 8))
 (segment (start 157.43 86.42) (end 157.43 90.74) (width 1.5) (layer B.Cu) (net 8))
 (segment (start 157.02 86.01) (end 157.43 86.42) (width 1.5) (layer B.Cu) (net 8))
 (segment (start 152.23 86.01) (end 152.23 87.29) (width 1.5) (layer B.Cu) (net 8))
 (segment (start 152.23 87.29) (end 151.26 88.26) (width 1.5) (layer B.Cu) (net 8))
 (segment (start 151.26 88.26) (end 142.77 88.26) (width 1.5) (layer B.Cu) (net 8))
 (segment (start 140.52 86.01) (end 135.68 86.01) (width 1.5) (layer B.Cu) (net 8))
 (segment (start 142.77 88.26) (end 140.52 86.01) (width 1.5) (layer B.Cu) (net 8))
 (segment (start 171.44 96.97) (end 173.67 96.97) (width 1.5) (layer B.Cu) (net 9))
 (segment (start 170.29 95.82) (end 171.44 96.97) (width 1.5) (layer B.Cu) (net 9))
 (segment (start 167.59 95.82) (end 170.29 95.82) (width 1.5) (layer B.Cu) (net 9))
 (segment (start 173.63 97.01) (end 173.67 96.97) (width 1.5) (layer B.Cu) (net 9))
 (segment (start 173.63 101.41) (end 173.63 97.01) (width 1.5) (layer B.Cu) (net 9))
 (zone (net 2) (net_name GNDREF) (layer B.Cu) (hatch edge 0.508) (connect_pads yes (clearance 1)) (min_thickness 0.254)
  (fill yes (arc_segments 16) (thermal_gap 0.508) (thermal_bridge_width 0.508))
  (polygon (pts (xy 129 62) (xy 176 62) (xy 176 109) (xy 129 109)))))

